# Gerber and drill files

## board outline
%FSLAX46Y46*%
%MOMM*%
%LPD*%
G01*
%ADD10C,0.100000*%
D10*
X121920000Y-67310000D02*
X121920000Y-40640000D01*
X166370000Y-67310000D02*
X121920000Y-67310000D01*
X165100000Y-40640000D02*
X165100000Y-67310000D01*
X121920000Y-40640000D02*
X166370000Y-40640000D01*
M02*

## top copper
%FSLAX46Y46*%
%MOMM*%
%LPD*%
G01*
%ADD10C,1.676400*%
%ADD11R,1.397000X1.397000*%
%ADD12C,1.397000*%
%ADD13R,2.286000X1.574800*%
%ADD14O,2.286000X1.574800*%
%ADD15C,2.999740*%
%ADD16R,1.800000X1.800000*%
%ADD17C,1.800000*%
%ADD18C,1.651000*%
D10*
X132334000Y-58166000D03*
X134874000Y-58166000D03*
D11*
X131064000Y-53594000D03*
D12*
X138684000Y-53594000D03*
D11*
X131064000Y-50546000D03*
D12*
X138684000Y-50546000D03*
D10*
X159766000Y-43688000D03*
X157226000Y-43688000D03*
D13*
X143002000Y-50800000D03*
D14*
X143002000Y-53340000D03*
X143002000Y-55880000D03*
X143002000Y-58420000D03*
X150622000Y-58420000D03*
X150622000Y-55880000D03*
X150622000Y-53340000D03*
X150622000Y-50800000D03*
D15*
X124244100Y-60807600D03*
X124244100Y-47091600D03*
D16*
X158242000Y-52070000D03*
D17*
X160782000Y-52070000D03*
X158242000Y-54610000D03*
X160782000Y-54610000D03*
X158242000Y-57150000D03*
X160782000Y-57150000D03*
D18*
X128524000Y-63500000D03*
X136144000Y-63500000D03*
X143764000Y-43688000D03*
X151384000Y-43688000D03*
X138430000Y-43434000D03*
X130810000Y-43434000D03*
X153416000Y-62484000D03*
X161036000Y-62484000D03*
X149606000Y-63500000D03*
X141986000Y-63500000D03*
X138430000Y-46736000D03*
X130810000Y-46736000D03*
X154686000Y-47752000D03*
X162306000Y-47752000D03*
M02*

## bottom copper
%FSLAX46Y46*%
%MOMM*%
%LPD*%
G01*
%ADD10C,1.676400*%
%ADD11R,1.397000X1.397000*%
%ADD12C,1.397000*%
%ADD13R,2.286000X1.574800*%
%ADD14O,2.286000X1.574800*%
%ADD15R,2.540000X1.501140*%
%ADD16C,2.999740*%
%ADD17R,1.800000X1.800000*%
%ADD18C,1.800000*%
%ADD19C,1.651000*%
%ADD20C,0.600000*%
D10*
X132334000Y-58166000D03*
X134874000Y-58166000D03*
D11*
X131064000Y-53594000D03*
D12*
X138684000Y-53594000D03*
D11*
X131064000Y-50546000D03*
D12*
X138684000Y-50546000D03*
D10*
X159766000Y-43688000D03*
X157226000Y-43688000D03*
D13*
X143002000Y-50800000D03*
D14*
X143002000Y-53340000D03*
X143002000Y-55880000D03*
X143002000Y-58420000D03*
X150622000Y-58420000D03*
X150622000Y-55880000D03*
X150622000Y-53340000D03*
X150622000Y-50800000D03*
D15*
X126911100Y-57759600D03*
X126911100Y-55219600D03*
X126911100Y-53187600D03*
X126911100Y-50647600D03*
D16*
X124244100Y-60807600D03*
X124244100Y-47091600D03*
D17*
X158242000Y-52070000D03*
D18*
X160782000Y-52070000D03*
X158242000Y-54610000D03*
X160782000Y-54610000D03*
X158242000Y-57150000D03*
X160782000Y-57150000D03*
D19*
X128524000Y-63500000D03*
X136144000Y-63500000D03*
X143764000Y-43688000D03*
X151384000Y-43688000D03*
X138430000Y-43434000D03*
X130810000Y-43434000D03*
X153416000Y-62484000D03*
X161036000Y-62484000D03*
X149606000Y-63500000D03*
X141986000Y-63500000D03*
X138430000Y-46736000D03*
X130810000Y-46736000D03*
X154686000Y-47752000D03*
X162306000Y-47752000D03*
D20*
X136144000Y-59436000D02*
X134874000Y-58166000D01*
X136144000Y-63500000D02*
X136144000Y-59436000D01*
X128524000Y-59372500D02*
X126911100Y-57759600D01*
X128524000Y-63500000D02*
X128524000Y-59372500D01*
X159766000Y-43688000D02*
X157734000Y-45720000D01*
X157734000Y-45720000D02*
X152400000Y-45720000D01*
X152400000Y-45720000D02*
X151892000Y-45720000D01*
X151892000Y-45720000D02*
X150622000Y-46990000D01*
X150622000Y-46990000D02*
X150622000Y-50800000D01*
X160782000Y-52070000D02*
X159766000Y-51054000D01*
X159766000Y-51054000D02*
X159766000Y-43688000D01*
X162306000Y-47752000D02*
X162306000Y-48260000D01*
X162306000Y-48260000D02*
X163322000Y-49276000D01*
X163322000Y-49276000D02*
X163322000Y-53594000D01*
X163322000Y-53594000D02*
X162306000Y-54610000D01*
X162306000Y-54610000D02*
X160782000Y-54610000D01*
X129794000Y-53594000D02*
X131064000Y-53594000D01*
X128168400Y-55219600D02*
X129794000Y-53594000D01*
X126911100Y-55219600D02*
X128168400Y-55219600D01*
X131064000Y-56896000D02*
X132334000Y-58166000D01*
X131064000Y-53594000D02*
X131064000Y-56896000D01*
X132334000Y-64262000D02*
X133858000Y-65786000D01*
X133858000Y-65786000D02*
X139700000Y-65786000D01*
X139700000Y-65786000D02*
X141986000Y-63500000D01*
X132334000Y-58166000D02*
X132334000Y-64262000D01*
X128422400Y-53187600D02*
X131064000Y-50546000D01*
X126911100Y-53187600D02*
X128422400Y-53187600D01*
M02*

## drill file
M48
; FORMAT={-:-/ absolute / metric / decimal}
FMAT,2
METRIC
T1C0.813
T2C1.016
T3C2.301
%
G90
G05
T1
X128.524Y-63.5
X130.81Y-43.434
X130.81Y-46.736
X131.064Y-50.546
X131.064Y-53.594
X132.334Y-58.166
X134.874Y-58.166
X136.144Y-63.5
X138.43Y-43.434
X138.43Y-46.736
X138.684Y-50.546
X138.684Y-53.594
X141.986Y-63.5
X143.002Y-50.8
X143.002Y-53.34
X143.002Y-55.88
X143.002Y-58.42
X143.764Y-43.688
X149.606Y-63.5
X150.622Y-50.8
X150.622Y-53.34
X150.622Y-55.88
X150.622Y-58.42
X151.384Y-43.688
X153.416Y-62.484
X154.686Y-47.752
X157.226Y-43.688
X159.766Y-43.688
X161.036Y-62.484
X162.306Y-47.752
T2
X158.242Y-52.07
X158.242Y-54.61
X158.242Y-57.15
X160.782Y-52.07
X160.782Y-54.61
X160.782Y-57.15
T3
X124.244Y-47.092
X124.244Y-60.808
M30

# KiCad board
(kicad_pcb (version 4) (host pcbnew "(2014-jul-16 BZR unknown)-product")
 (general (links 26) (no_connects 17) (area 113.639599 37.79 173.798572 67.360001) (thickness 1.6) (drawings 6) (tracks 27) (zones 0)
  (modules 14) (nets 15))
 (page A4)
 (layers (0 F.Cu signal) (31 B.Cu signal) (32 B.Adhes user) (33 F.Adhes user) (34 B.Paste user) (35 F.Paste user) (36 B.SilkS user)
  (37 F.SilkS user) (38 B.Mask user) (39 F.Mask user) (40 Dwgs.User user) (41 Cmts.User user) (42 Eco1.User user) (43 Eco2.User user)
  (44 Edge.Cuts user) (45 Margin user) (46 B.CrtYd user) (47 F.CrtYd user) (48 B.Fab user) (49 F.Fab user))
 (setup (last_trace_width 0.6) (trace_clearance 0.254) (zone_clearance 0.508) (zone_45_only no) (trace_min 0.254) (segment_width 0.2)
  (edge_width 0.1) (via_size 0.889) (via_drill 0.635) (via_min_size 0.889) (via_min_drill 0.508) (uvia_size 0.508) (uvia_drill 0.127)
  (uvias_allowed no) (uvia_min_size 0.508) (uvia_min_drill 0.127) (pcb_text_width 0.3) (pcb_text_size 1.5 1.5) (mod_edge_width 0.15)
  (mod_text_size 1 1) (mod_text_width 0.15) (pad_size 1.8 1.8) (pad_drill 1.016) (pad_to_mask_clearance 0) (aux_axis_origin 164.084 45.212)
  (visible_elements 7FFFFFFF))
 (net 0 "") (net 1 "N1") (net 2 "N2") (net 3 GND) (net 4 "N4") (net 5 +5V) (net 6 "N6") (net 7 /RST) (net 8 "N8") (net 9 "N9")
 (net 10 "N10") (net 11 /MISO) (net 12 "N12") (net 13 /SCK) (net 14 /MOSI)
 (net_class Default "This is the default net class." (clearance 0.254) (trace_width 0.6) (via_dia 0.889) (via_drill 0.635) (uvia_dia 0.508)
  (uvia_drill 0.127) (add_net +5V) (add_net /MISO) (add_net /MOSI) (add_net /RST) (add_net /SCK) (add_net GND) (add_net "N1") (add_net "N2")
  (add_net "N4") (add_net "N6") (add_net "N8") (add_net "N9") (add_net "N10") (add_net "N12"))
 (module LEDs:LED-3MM (layer F.Cu) (at 133.604 58.166)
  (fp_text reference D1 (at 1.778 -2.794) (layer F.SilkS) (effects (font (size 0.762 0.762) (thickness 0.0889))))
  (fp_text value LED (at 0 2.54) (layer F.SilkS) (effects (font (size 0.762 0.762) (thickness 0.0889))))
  (pad 1 thru_hole circle (at -1.27 0) (size 1.6764 1.6764) (drill 0.8128) (layers *.Cu *.Mask F.SilkS) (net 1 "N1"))
  (pad 2 thru_hole circle (at 1.27 0) (size 1.6764 1.6764) (drill 0.8128) (layers *.Cu *.Mask F.SilkS) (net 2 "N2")))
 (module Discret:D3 (layer F.Cu) (at 134.874 53.594 180)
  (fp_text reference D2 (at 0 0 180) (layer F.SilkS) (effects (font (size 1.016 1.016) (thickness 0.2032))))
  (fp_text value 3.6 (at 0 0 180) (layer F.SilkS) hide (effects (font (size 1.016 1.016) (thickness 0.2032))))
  (pad 2 thru_hole rect (at 3.81 0 180) (size 1.397 1.397) (drill 0.8128) (layers *.Cu *.Mask F.SilkS) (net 1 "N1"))
  (pad 1 thru_hole circle (at -3.81 0 180) (size 1.397 1.397) (drill 0.8128) (layers *.Cu *.Mask F.SilkS) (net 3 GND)))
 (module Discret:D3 (layer F.Cu) (at 134.874 50.546 180)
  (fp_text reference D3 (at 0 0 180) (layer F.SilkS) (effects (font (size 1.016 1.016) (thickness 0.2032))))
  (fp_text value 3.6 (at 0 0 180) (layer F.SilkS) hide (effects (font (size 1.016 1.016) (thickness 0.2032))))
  (pad 2 thru_hole rect (at 3.81 0 180) (size 1.397 1.397) (drill 0.8128) (layers *.Cu *.Mask F.SilkS) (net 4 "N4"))
  (pad 1 thru_hole circle (at -3.81 0 180) (size 1.397 1.397) (drill 0.8128) (layers *.Cu *.Mask F.SilkS) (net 3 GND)))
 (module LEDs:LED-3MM (layer F.Cu) (at 158.496 43.688 180)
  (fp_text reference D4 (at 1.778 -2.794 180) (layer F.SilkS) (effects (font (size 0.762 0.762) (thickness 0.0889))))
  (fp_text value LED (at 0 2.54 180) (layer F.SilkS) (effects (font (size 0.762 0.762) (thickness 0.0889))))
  (pad 1 thru_hole circle (at -1.27 0 180) (size 1.6764 1.6764) (drill 0.8128) (layers *.Cu *.Mask F.SilkS) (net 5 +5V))
  (pad 2 thru_hole circle (at 1.27 0 180) (size 1.6764 1.6764) (drill 0.8128) (layers *.Cu *.Mask F.SilkS) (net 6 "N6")))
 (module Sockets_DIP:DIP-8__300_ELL (layer F.Cu) (at 146.812 54.61 270)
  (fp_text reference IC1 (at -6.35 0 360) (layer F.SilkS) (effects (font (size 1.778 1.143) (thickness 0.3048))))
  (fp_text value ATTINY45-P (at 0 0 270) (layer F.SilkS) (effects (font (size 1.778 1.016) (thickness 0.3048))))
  (pad 1 thru_hole rect (at -3.81 3.81 270) (size 1.5748 2.286) (drill 0.8128) (layers *.Cu *.Mask F.SilkS) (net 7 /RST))
  (pad 2 thru_hole oval (at -1.27 3.81 270) (size 1.5748 2.286) (drill 0.8128) (layers *.Cu *.Mask F.SilkS) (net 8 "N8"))
  (pad 3 thru_hole oval (at 1.27 3.81 270) (size 1.5748 2.286) (drill 0.8128) (layers *.Cu *.Mask F.SilkS) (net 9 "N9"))
  (pad 4 thru_hole oval (at 3.81 3.81 270) (size 1.5748 2.286) (drill 0.8128) (layers *.Cu *.Mask F.SilkS) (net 3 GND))
  (pad 5 thru_hole oval (at 3.81 -3.81 270) (size 1.5748 2.286) (drill 0.8128) (layers *.Cu *.Mask F.SilkS) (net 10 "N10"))
  (pad 6 thru_hole oval (at 1.27 -3.81 270) (size 1.5748 2.286) (drill 0.8128) (layers *.Cu *.Mask F.SilkS) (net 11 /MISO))
  (pad 7 thru_hole oval (at -1.27 -3.81 270) (size 1.5748 2.286) (drill 0.8128) (layers *.Cu *.Mask F.SilkS) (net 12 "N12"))
  (pad 8 thru_hole oval (at -3.81 -3.81 270) (size 1.5748 2.286) (drill 0.8128) (layers *.Cu *.Mask F.SilkS) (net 5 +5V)))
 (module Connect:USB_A (layer F.Cu) (at 126.9111 54.2036 180)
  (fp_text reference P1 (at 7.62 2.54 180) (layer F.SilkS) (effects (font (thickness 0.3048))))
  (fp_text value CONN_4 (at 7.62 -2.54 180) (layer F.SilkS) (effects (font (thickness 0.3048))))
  (pad 4 smd rect (at 0 -3.556 180) (size 2.54 1.50114) (layers B.Cu F.Paste F.Mask) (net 3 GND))
  (pad 3 smd rect (at 0 -1.016 180) (size 2.54 1.50114) (layers B.Cu F.Paste F.Mask) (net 1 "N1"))
  (pad 2 smd rect (at 0 1.016 180) (size 2.54 1.50114) (layers B.Cu F.Paste F.Mask) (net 4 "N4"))
  (pad 1 smd rect (at 0 3.556 180) (size 2.54 1.50114) (layers B.Cu F.Paste F.Mask) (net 5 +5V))
  (pad 5 thru_hole circle (at 2.667 -6.604 180) (size 2.99974 2.99974) (drill 2.30124) (layers *.Cu *.Mask F.SilkS))
  (pad 6 thru_hole circle (at 2.667 7.112 180) (size 2.99974 2.99974) (drill 2.30124) (layers *.Cu *.Mask F.SilkS)))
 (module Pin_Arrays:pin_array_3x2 (layer F.Cu) (at 159.512 54.61 270)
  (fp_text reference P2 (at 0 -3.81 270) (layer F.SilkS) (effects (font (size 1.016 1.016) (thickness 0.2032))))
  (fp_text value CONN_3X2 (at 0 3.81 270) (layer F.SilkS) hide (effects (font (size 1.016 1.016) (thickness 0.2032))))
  (pad 1 thru_hole rect (at -2.54 1.27 270) (size 1.8 1.8) (drill 1.016) (layers *.Cu *.Mask F.SilkS) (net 11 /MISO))
  (pad 2 thru_hole circle (at -2.54 -1.27 270) (size 1.8 1.8) (drill 1.016) (layers *.Cu *.Mask F.SilkS) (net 5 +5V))
  (pad 3 thru_hole circle (at 0 1.27 270) (size 1.8 1.8) (drill 1.016) (layers *.Cu *.Mask F.SilkS) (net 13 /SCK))
  (pad 4 thru_hole circle (at 0 -1.27 270) (size 1.8 1.8) (drill 1.016) (layers *.Cu *.Mask F.SilkS) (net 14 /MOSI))
  (pad e thru_hole circle (at 2.54 1.27 270) (size 1.8 1.8) (drill 1.016) (layers *.Cu *.Mask F.SilkS) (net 7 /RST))
  (pad 6 thru_hole circle (at 2.54 -1.27 270) (size 1.8 1.8) (drill 1.016) (layers *.Cu *.Mask F.SilkS) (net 3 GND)))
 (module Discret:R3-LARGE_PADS (layer F.Cu) (at 132.334 63.5) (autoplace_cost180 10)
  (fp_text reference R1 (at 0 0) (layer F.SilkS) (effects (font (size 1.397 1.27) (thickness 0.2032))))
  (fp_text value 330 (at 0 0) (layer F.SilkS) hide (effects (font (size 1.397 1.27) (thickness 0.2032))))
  (pad 1 thru_hole circle (at -3.81 0) (size 1.651 1.651) (drill 0.8128) (layers *.Cu *.Mask F.SilkS) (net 3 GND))
  (pad 2 thru_hole circle (at 3.81 0) (size 1.651 1.651) (drill 0.8128) (layers *.Cu *.Mask F.SilkS) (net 2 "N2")))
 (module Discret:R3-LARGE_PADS (layer F.Cu) (at 147.574 43.688) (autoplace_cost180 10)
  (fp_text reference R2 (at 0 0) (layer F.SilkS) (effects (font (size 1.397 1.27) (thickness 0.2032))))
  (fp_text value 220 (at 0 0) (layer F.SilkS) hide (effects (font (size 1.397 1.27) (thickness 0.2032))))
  (pad 1 thru_hole circle (at -3.81 0) (size 1.651 1.651) (drill 0.8128) (layers *.Cu *.Mask F.SilkS) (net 3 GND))
  (pad 2 thru_hole circle (at 3.81 0) (size 1.651 1.651) (drill 0.8128) (layers *.Cu *.Mask F.SilkS) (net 6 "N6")))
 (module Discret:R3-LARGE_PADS (layer F.Cu) (at 134.62 43.434 180) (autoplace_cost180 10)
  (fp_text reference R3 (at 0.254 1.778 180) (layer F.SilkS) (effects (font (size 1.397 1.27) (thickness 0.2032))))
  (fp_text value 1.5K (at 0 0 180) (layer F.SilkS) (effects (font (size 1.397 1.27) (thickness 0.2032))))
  (pad 1 thru_hole circle (at -3.81 0 180) (size 1.651 1.651) (drill 0.8128) (layers *.Cu *.Mask F.SilkS) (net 5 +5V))
  (pad 2 thru_hole circle (at 3.81 0 180) (size 1.651 1.651) (drill 0.8128) (layers *.Cu *.Mask F.SilkS) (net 4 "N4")))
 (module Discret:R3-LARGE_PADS (layer F.Cu) (at 157.226 62.484) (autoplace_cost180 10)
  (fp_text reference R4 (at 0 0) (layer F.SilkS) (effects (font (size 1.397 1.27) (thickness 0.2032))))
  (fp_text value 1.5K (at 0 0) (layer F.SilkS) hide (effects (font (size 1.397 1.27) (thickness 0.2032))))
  (pad 1 thru_hole circle (at -3.81 0) (size 1.651 1.651) (drill 0.8128) (layers *.Cu *.Mask F.SilkS) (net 12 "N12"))
  (pad 2 thru_hole circle (at 3.81 0) (size 1.651 1.651) (drill 0.8128) (layers *.Cu *.Mask F.SilkS) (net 13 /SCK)))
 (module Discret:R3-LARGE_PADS (layer F.Cu) (at 145.796 63.5 180) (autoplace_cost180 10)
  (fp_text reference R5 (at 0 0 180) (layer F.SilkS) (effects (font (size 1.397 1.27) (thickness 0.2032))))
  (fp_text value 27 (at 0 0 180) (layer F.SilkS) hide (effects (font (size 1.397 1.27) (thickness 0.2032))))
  (pad 1 thru_hole circle (at -3.81 0 180) (size 1.651 1.651) (drill 0.8128) (layers *.Cu *.Mask F.SilkS) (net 8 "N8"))
  (pad 2 thru_hole circle (at 3.81 0 180) (size 1.651 1.651) (drill 0.8128) (layers *.Cu *.Mask F.SilkS) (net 1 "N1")))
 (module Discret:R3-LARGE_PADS (layer F.Cu) (at 134.62 46.736 180) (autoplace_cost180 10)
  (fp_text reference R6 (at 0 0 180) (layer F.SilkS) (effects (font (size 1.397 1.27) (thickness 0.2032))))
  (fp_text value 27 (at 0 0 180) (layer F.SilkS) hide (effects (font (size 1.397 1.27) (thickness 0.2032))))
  (pad 1 thru_hole circle (at -3.81 0 180) (size 1.651 1.651) (drill 0.8128) (layers *.Cu *.Mask F.SilkS) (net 9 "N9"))
  (pad 2 thru_hole circle (at 3.81 0 180) (size 1.651 1.651) (drill 0.8128) (layers *.Cu *.Mask F.SilkS) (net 4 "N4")))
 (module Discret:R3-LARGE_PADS (layer F.Cu) (at 158.496 47.752) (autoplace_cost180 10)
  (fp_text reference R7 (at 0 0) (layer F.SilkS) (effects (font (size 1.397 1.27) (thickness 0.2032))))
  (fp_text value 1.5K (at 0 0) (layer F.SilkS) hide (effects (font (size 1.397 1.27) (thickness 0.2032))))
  (pad 1 thru_hole circle (at -3.81 0) (size 1.651 1.651) (drill 0.8128) (layers *.Cu *.Mask F.SilkS) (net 10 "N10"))
  (pad 2 thru_hole circle (at 3.81 0) (size 1.651 1.651) (drill 0.8128) (layers *.Cu *.Mask F.SilkS) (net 14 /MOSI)))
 (gr_line (start 121.92 67.31) (end 121.92 40.64) (angle 90) (layer Edge.Cuts) (width 0.1))
 (gr_line (start 166.37 67.31) (end 121.92 67.31) (angle 90) (layer Edge.Cuts) (width 0.1))
 (gr_line (start 165.1 40.64) (end 165.1 67.31) (angle 90) (layer Edge.Cuts) (width 0.1))
 (gr_line (start 121.92 40.64) (end 166.37 40.64) (angle 90) (layer Edge.Cuts) (width 0.1))
 (segment (start 136.144 59.436) (end 134.874 58.166) (width 0.6) (layer B.Cu) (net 2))
 (segment (start 136.144 63.5) (end 136.144 59.436) (width 0.6) (layer B.Cu) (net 2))
 (segment (start 128.524 59.3725) (end 126.9111 57.7596) (width 0.6) (layer B.Cu) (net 3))
 (segment (start 128.524 63.5) (end 128.524 59.3725) (width 0.6) (layer B.Cu) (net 3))
 (segment (start 159.766 43.688) (end 157.734 45.72) (width 0.6) (layer B.Cu) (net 5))
 (segment (start 157.734 45.72) (end 152.4 45.72) (width 0.6) (layer B.Cu) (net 5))
 (segment (start 152.4 45.72) (end 151.892 45.72) (width 0.6) (layer B.Cu) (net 5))
 (segment (start 151.892 45.72) (end 150.622 46.99) (width 0.6) (layer B.Cu) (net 5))
 (segment (start 150.622 46.99) (end 150.622 50.8) (width 0.6) (layer B.Cu) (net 5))
 (segment (start 160.782 52.07) (end 159.766 51.054) (width 0.6) (layer B.Cu) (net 5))
 (segment (start 159.766 51.054) (end 159.766 43.688) (width 0.6) (layer B.Cu) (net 5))
 (segment (start 162.306 47.752) (end 162.306 48.26) (width 0.6) (layer B.Cu) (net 14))
 (segment (start 162.306 48.26) (end 163.322 49.276) (width 0.6) (layer B.Cu) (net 14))
 (segment (start 163.322 49.276) (end 163.322 53.594) (width 0.6) (layer B.Cu) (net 14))
 (segment (start 163.322 53.594) (end 162.306 54.61) (width 0.6) (layer B.Cu) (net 14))
 (segment (start 162.306 54.61) (end 160.782 54.61) (width 0.6) (layer B.Cu) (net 14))
 (segment (start 129.794 53.594) (end 131.064 53.594) (width 0.6) (layer B.Cu) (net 1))
 (segment (start 128.1684 55.2196) (end 129.794 53.594) (width 0.6) (layer B.Cu) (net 1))
 (segment (start 126.9111 55.2196) (end 128.1684 55.2196) (width 0.6) (layer B.Cu) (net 1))
 (segment (start 131.064 56.896) (end 132.334 58.166) (width 0.6) (layer B.Cu) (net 1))
 (segment (start 131.064 53.594) (end 131.064 56.896) (width 0.6) (layer B.Cu) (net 1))
 (segment (start 132.334 64.262) (end 133.858 65.786) (width 0.6) (layer B.Cu) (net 1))
 (segment (start 133.858 65.786) (end 139.7 65.786) (width 0.6) (layer B.Cu) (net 1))
 (segment (start 139.7 65.786) (end 141.986 63.5) (width 0.6) (layer B.Cu) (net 1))
 (segment (start 132.334 58.166) (end 132.334 64.262) (width 0.6) (layer B.Cu) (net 1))
 (segment (start 128.4224 53.1876) (end 131.064 50.546) (width 0.6) (layer B.Cu) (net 4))
 (segment (start 126.9111 53.1876) (end 128.4224 53.1876) (width 0.6) (layer B.Cu) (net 4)))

